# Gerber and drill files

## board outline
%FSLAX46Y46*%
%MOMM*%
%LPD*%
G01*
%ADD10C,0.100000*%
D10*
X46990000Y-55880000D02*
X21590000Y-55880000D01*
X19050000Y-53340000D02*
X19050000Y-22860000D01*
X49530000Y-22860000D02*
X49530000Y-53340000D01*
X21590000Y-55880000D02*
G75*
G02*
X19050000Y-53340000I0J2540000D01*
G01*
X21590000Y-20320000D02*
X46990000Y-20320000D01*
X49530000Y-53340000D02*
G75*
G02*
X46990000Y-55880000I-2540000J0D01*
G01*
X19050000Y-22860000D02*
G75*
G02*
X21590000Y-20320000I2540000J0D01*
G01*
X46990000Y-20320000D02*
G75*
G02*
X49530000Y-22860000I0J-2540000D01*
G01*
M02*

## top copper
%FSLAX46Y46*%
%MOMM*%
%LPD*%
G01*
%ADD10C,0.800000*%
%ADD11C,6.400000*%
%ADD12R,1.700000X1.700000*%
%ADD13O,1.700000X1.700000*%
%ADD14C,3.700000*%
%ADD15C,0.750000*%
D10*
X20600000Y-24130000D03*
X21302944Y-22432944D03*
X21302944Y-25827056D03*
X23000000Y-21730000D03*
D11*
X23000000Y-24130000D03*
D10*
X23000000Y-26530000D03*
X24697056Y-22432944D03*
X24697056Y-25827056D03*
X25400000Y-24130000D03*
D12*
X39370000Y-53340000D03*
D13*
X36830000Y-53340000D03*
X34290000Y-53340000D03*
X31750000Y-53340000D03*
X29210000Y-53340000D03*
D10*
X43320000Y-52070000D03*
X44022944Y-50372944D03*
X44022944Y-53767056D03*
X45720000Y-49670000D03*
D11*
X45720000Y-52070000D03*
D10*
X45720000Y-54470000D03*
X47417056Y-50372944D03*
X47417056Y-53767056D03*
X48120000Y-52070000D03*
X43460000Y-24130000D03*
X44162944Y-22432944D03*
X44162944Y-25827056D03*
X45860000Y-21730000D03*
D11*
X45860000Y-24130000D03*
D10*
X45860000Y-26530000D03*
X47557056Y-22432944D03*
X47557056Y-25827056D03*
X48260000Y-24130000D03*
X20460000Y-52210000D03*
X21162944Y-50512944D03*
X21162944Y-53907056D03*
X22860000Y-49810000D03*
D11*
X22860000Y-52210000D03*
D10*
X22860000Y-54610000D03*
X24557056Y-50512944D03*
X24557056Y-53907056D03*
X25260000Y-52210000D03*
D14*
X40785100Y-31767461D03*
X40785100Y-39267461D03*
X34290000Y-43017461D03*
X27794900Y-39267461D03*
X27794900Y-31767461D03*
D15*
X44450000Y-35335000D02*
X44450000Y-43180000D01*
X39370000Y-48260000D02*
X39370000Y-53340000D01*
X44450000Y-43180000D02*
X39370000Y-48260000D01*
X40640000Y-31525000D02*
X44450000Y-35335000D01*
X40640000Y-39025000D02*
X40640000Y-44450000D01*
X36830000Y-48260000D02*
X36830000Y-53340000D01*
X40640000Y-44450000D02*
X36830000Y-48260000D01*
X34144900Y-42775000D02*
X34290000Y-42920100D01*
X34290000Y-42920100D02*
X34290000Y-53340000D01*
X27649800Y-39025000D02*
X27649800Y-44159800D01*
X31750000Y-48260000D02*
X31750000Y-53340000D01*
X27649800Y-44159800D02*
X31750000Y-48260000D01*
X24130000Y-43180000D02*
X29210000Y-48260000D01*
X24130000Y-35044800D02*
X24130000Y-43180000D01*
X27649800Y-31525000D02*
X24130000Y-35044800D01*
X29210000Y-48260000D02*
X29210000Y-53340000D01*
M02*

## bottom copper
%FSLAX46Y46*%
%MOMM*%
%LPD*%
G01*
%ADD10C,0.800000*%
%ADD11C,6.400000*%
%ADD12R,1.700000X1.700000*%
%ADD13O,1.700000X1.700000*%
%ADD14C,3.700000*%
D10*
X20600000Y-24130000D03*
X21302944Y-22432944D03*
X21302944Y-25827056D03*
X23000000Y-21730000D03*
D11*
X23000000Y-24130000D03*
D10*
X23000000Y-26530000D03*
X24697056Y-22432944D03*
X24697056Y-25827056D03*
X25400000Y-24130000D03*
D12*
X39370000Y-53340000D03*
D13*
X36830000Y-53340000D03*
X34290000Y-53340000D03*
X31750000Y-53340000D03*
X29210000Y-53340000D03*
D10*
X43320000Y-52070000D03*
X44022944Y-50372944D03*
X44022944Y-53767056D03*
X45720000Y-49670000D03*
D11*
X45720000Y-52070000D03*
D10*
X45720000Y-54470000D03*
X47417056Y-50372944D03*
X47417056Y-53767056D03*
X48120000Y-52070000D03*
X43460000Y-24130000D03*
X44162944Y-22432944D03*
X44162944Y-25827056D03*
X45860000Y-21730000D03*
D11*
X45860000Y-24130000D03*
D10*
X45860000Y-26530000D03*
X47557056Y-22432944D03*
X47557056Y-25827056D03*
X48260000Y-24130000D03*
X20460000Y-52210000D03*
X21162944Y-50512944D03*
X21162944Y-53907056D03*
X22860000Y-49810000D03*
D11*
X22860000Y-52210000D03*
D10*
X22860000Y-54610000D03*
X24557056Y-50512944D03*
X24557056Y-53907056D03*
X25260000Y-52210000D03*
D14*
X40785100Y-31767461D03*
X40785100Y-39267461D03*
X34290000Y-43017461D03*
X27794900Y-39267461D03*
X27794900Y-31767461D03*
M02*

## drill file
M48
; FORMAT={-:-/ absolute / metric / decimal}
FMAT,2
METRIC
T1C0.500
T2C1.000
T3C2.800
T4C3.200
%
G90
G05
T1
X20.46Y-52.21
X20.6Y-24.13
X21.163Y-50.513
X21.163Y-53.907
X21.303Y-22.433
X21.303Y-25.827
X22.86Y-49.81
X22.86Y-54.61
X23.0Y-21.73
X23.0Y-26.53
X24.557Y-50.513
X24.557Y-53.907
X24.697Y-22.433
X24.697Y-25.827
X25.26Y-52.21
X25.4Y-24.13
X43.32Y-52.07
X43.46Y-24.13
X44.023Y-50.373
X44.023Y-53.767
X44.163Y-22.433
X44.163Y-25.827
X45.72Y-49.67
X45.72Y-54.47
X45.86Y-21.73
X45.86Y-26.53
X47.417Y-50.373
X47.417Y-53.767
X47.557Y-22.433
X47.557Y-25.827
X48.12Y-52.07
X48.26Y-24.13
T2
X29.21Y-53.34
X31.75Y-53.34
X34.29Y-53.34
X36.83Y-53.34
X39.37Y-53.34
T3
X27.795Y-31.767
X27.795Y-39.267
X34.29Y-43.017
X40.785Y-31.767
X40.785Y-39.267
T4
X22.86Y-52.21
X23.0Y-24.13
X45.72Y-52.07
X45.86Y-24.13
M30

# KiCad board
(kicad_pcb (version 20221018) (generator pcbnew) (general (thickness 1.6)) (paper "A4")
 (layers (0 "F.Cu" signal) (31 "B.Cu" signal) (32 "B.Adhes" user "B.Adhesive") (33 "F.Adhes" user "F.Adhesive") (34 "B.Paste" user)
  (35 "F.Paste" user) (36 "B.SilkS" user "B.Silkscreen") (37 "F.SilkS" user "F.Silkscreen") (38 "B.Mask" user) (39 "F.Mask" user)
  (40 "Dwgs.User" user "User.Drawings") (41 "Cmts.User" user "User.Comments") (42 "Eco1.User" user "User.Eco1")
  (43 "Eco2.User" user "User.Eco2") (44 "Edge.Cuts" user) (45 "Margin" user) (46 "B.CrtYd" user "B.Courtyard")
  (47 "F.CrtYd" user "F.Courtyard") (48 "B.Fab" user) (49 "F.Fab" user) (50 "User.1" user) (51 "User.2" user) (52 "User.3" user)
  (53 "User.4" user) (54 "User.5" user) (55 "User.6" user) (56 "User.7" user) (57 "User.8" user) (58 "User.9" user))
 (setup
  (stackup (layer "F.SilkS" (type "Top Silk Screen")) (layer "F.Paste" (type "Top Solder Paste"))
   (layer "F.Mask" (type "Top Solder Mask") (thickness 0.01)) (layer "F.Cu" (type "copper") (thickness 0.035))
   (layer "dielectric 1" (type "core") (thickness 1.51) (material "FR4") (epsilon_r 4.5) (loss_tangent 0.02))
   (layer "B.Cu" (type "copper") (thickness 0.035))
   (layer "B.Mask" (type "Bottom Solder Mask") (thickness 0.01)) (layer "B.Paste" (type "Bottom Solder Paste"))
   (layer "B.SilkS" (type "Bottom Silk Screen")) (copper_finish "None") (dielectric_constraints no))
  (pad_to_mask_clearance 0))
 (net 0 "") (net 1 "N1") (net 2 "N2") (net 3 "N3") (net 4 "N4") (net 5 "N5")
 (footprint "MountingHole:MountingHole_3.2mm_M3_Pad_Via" (layer "F.Cu") (at 23 24.13)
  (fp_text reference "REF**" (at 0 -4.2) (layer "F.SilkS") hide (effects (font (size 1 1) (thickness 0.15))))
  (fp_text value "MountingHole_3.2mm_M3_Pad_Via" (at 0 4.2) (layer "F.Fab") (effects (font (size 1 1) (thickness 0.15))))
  (pad "1" thru_hole circle (at -2.4 0) (size 0.8 0.8) (drill 0.5) (layers "*.Cu" "*.Mask") (zone_connect 2))
  (pad "1" thru_hole circle (at -1.697056 -1.697056) (size 0.8 0.8) (drill 0.5) (layers "*.Cu" "*.Mask") (zone_connect 2))
  (pad "1" thru_hole circle (at -1.697056 1.697056) (size 0.8 0.8) (drill 0.5) (layers "*.Cu" "*.Mask") (zone_connect 2))
  (pad "1" thru_hole circle (at 0 -2.4) (size 0.8 0.8) (drill 0.5) (layers "*.Cu" "*.Mask") (zone_connect 2))
  (pad "1" thru_hole circle (at 0 0) (size 6.4 6.4) (drill 3.2) (layers "*.Cu" "*.Mask"))
  (pad "1" thru_hole circle (at 0 2.4) (size 0.8 0.8) (drill 0.5) (layers "*.Cu" "*.Mask") (zone_connect 2))
  (pad "1" thru_hole circle (at 1.697056 -1.697056) (size 0.8 0.8) (drill 0.5) (layers "*.Cu" "*.Mask") (zone_connect 2))
  (pad "1" thru_hole circle (at 1.697056 1.697056) (size 0.8 0.8) (drill 0.5) (layers "*.Cu" "*.Mask") (zone_connect 2))
  (pad "1" thru_hole circle (at 2.4 0) (size 0.8 0.8) (drill 0.5) (layers "*.Cu" "*.Mask") (zone_connect 2)))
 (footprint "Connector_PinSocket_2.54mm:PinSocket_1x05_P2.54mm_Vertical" (layer "F.Cu") (at 39.37 53.34 -90)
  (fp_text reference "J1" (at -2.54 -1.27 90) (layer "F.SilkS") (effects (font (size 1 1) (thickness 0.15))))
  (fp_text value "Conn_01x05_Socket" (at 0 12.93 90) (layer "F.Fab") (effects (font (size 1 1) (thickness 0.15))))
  (pad "1" thru_hole rect (at 0 0 270) (size 1.7 1.7) (drill 1) (layers "*.Cu" "*.Mask") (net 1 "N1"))
  (pad "2" thru_hole oval (at 0 2.54 270) (size 1.7 1.7) (drill 1) (layers "*.Cu" "*.Mask") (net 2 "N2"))
  (pad "3" thru_hole oval (at 0 5.08 270) (size 1.7 1.7) (drill 1) (layers "*.Cu" "*.Mask") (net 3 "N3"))
  (pad "4" thru_hole oval (at 0 7.62 270) (size 1.7 1.7) (drill 1) (layers "*.Cu" "*.Mask") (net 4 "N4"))
  (pad "5" thru_hole oval (at 0 10.16 270) (size 1.7 1.7) (drill 1) (layers "*.Cu" "*.Mask") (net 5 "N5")))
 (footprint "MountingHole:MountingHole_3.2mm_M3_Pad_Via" (layer "F.Cu") (at 45.72 52.07)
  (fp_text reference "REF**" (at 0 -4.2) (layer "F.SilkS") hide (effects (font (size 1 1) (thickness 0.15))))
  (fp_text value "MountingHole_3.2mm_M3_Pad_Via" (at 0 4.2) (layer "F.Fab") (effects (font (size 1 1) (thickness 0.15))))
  (pad "1" thru_hole circle (at -2.4 0) (size 0.8 0.8) (drill 0.5) (layers "*.Cu" "*.Mask") (zone_connect 2))
  (pad "1" thru_hole circle (at -1.697056 -1.697056) (size 0.8 0.8) (drill 0.5) (layers "*.Cu" "*.Mask") (zone_connect 2))
  (pad "1" thru_hole circle (at -1.697056 1.697056) (size 0.8 0.8) (drill 0.5) (layers "*.Cu" "*.Mask") (zone_connect 2))
  (pad "1" thru_hole circle (at 0 -2.4) (size 0.8 0.8) (drill 0.5) (layers "*.Cu" "*.Mask") (zone_connect 2))
  (pad "1" thru_hole circle (at 0 0) (size 6.4 6.4) (drill 3.2) (layers "*.Cu" "*.Mask"))
  (pad "1" thru_hole circle (at 0 2.4) (size 0.8 0.8) (drill 0.5) (layers "*.Cu" "*.Mask") (zone_connect 2))
  (pad "1" thru_hole circle (at 1.697056 -1.697056) (size 0.8 0.8) (drill 0.5) (layers "*.Cu" "*.Mask") (zone_connect 2))
  (pad "1" thru_hole circle (at 1.697056 1.697056) (size 0.8 0.8) (drill 0.5) (layers "*.Cu" "*.Mask") (zone_connect 2))
  (pad "1" thru_hole circle (at 2.4 0) (size 0.8 0.8) (drill 0.5) (layers "*.Cu" "*.Mask") (zone_connect 2)))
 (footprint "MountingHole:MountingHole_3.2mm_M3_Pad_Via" (layer "F.Cu") (at 45.86 24.13)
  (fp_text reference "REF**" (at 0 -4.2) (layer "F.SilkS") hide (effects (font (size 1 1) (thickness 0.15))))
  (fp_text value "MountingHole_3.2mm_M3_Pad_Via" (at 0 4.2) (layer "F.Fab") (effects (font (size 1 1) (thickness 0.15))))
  (pad "1" thru_hole circle (at -2.4 0) (size 0.8 0.8) (drill 0.5) (layers "*.Cu" "*.Mask") (zone_connect 2))
  (pad "1" thru_hole circle (at -1.697056 -1.697056) (size 0.8 0.8) (drill 0.5) (layers "*.Cu" "*.Mask") (zone_connect 2))
  (pad "1" thru_hole circle (at -1.697056 1.697056) (size 0.8 0.8) (drill 0.5) (layers "*.Cu" "*.Mask") (zone_connect 2))
  (pad "1" thru_hole circle (at 0 -2.4) (size 0.8 0.8) (drill 0.5) (layers "*.Cu" "*.Mask") (zone_connect 2))
  (pad "1" thru_hole circle (at 0 0) (size 6.4 6.4) (drill 3.2) (layers "*.Cu" "*.Mask"))
  (pad "1" thru_hole circle (at 0 2.4) (size 0.8 0.8) (drill 0.5) (layers "*.Cu" "*.Mask") (zone_connect 2))
  (pad "1" thru_hole circle (at 1.697056 -1.697056) (size 0.8 0.8) (drill 0.5) (layers "*.Cu" "*.Mask") (zone_connect 2))
  (pad "1" thru_hole circle (at 1.697056 1.697056) (size 0.8 0.8) (drill 0.5) (layers "*.Cu" "*.Mask") (zone_connect 2))
  (pad "1" thru_hole circle (at 2.4 0) (size 0.8 0.8) (drill 0.5) (layers "*.Cu" "*.Mask") (zone_connect 2)))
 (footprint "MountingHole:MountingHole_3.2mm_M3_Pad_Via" (layer "F.Cu") (at 22.86 52.21)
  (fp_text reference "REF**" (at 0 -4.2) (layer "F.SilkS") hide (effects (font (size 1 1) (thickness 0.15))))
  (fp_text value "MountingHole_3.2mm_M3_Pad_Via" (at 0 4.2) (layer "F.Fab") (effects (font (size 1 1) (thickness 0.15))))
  (pad "1" thru_hole circle (at -2.4 0) (size 0.8 0.8) (drill 0.5) (layers "*.Cu" "*.Mask") (zone_connect 2))
  (pad "1" thru_hole circle (at -1.697056 -1.697056) (size 0.8 0.8) (drill 0.5) (layers "*.Cu" "*.Mask") (zone_connect 2))
  (pad "1" thru_hole circle (at -1.697056 1.697056) (size 0.8 0.8) (drill 0.5) (layers "*.Cu" "*.Mask") (zone_connect 2))
  (pad "1" thru_hole circle (at 0 -2.4) (size 0.8 0.8) (drill 0.5) (layers "*.Cu" "*.Mask") (zone_connect 2))
  (pad "1" thru_hole circle (at 0 0) (size 6.4 6.4) (drill 3.2) (layers "*.Cu" "*.Mask"))
  (pad "1" thru_hole circle (at 0 2.4) (size 0.8 0.8) (drill 0.5) (layers "*.Cu" "*.Mask") (zone_connect 2))
  (pad "1" thru_hole circle (at 1.697056 -1.697056) (size 0.8 0.8) (drill 0.5) (layers "*.Cu" "*.Mask") (zone_connect 2))
  (pad "1" thru_hole circle (at 1.697056 1.697056) (size 0.8 0.8) (drill 0.5) (layers "*.Cu" "*.Mask") (zone_connect 2))
  (pad "1" thru_hole circle (at 2.4 0) (size 0.8 0.8) (drill 0.5) (layers "*.Cu" "*.Mask") (zone_connect 2)))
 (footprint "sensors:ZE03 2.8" (layer "F.Cu") (at 34.29 35.517461)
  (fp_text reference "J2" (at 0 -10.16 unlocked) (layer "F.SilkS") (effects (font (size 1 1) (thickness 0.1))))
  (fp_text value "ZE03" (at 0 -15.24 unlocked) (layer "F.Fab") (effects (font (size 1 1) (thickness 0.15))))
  (pad "1" thru_hole circle (at 6.4951 -3.75) (size 3.7 3.7) (drill 2.8) (layers "*.Cu" "*.Mask") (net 1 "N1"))
  (pad "2" thru_hole circle (at 6.4951 3.75) (size 3.7 3.7) (drill 2.8) (layers "*.Cu" "*.Mask") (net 2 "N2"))
  (pad "3" thru_hole circle (at 0 7.5) (size 3.7 3.7) (drill 2.8) (layers "*.Cu" "*.Mask") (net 3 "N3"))
  (pad "4" thru_hole circle (at -6.4951 3.75) (size 3.7 3.7) (drill 2.8) (layers "*.Cu" "*.Mask") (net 4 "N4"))
  (pad "5" thru_hole circle (at -6.4951 -3.75) (size 3.7 3.7) (drill 2.8) (layers "*.Cu" "*.Mask") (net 5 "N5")))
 (gr_line (start 46.99 55.88) (end 21.59 55.88) (stroke (width 0.1) (type default)) (layer "Edge.Cuts"))
 (gr_line (start 19.05 53.34) (end 19.05 22.86) (stroke (width 0.1) (type default)) (layer "Edge.Cuts"))
 (gr_line (start 49.53 22.86) (end 49.53 53.34) (stroke (width 0.1) (type default)) (layer "Edge.Cuts"))
 (gr_arc (start 21.59 55.88) (mid 19.793949 55.136051) (end 19.05 53.34) (stroke (width 0.1) (type default)) (layer "Edge.Cuts"))
 (gr_line (start 21.59 20.32) (end 46.99 20.32) (stroke (width 0.1) (type default)) (layer "Edge.Cuts"))
 (gr_arc (start 49.53 53.34) (mid 48.786051 55.136051) (end 46.99 55.88) (stroke (width 0.1) (type default)) (layer "Edge.Cuts"))
 (gr_arc (start 19.05 22.86) (mid 19.793949 21.063949) (end 21.59 20.32) (stroke (width 0.1) (type default)) (layer "Edge.Cuts"))
 (gr_arc (start 46.99 20.32) (mid 48.786051 21.063949) (end 49.53 22.86) (stroke (width 0.1) (type default)) (layer "Edge.Cuts"))
 (segment (start 44.45 35.335) (end 44.45 43.18) (width 0.75) (layer "F.Cu") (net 1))
 (segment (start 39.37 48.26) (end 39.37 53.34) (width 0.75) (layer "F.Cu") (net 1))
 (segment (start 44.45 43.18) (end 39.37 48.26) (width 0.75) (layer "F.Cu") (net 1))
 (segment (start 40.64 31.525) (end 44.45 35.335) (width 0.75) (layer "F.Cu") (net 1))
 (segment (start 40.64 39.025) (end 40.64 44.45) (width 0.75) (layer "F.Cu") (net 2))
 (segment (start 36.83 48.26) (end 36.83 53.34) (width 0.75) (layer "F.Cu") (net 2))
 (segment (start 40.64 44.45) (end 36.83 48.26) (width 0.75) (layer "F.Cu") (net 2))
 (segment (start 34.1449 42.775) (end 34.29 42.9201) (width 0.75) (layer "F.Cu") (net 3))
 (segment (start 34.29 42.9201) (end 34.29 53.34) (width 0.75) (layer "F.Cu") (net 3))
 (segment (start 27.6498 39.025) (end 27.6498 44.1598) (width 0.75) (layer "F.Cu") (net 4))
 (segment (start 31.75 48.26) (end 31.75 53.34) (width 0.75) (layer "F.Cu") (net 4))
 (segment (start 27.6498 44.1598) (end 31.75 48.26) (width 0.75) (layer "F.Cu") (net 4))
 (segment (start 24.13 43.18) (end 29.21 48.26) (width 0.75) (layer "F.Cu") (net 5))
 (segment (start 24.13 35.0448) (end 24.13 43.18) (width 0.75) (layer "F.Cu") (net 5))
 (segment (start 27.6498 31.525) (end 24.13 35.0448) (width 0.75) (layer "F.Cu") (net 5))
 (segment (start 29.21 48.26) (end 29.21 53.34) (width 0.75) (layer "F.Cu") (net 5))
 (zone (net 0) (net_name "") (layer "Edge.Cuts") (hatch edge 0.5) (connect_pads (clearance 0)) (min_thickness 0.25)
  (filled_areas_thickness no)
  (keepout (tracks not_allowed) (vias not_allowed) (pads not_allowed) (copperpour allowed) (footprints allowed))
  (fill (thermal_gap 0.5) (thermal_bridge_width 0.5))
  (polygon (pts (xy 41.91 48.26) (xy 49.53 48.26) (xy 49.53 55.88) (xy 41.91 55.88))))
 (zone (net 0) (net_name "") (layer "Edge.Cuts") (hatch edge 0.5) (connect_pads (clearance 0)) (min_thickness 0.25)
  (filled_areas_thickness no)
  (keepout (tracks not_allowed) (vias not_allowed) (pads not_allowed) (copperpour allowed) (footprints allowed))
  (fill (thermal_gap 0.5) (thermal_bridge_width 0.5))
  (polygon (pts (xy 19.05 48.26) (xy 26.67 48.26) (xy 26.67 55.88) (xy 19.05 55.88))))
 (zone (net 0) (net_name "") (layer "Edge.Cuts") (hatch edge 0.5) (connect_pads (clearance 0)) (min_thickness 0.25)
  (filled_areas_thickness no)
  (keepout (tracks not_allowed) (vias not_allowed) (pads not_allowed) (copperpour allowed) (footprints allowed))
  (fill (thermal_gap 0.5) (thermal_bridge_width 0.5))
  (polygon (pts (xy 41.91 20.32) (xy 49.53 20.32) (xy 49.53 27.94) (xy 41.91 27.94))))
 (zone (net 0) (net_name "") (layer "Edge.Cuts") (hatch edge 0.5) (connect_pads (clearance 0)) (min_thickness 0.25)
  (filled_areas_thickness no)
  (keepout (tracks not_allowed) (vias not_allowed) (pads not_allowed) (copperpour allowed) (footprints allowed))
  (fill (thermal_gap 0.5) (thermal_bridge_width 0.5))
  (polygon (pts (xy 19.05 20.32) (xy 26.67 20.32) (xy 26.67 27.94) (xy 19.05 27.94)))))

